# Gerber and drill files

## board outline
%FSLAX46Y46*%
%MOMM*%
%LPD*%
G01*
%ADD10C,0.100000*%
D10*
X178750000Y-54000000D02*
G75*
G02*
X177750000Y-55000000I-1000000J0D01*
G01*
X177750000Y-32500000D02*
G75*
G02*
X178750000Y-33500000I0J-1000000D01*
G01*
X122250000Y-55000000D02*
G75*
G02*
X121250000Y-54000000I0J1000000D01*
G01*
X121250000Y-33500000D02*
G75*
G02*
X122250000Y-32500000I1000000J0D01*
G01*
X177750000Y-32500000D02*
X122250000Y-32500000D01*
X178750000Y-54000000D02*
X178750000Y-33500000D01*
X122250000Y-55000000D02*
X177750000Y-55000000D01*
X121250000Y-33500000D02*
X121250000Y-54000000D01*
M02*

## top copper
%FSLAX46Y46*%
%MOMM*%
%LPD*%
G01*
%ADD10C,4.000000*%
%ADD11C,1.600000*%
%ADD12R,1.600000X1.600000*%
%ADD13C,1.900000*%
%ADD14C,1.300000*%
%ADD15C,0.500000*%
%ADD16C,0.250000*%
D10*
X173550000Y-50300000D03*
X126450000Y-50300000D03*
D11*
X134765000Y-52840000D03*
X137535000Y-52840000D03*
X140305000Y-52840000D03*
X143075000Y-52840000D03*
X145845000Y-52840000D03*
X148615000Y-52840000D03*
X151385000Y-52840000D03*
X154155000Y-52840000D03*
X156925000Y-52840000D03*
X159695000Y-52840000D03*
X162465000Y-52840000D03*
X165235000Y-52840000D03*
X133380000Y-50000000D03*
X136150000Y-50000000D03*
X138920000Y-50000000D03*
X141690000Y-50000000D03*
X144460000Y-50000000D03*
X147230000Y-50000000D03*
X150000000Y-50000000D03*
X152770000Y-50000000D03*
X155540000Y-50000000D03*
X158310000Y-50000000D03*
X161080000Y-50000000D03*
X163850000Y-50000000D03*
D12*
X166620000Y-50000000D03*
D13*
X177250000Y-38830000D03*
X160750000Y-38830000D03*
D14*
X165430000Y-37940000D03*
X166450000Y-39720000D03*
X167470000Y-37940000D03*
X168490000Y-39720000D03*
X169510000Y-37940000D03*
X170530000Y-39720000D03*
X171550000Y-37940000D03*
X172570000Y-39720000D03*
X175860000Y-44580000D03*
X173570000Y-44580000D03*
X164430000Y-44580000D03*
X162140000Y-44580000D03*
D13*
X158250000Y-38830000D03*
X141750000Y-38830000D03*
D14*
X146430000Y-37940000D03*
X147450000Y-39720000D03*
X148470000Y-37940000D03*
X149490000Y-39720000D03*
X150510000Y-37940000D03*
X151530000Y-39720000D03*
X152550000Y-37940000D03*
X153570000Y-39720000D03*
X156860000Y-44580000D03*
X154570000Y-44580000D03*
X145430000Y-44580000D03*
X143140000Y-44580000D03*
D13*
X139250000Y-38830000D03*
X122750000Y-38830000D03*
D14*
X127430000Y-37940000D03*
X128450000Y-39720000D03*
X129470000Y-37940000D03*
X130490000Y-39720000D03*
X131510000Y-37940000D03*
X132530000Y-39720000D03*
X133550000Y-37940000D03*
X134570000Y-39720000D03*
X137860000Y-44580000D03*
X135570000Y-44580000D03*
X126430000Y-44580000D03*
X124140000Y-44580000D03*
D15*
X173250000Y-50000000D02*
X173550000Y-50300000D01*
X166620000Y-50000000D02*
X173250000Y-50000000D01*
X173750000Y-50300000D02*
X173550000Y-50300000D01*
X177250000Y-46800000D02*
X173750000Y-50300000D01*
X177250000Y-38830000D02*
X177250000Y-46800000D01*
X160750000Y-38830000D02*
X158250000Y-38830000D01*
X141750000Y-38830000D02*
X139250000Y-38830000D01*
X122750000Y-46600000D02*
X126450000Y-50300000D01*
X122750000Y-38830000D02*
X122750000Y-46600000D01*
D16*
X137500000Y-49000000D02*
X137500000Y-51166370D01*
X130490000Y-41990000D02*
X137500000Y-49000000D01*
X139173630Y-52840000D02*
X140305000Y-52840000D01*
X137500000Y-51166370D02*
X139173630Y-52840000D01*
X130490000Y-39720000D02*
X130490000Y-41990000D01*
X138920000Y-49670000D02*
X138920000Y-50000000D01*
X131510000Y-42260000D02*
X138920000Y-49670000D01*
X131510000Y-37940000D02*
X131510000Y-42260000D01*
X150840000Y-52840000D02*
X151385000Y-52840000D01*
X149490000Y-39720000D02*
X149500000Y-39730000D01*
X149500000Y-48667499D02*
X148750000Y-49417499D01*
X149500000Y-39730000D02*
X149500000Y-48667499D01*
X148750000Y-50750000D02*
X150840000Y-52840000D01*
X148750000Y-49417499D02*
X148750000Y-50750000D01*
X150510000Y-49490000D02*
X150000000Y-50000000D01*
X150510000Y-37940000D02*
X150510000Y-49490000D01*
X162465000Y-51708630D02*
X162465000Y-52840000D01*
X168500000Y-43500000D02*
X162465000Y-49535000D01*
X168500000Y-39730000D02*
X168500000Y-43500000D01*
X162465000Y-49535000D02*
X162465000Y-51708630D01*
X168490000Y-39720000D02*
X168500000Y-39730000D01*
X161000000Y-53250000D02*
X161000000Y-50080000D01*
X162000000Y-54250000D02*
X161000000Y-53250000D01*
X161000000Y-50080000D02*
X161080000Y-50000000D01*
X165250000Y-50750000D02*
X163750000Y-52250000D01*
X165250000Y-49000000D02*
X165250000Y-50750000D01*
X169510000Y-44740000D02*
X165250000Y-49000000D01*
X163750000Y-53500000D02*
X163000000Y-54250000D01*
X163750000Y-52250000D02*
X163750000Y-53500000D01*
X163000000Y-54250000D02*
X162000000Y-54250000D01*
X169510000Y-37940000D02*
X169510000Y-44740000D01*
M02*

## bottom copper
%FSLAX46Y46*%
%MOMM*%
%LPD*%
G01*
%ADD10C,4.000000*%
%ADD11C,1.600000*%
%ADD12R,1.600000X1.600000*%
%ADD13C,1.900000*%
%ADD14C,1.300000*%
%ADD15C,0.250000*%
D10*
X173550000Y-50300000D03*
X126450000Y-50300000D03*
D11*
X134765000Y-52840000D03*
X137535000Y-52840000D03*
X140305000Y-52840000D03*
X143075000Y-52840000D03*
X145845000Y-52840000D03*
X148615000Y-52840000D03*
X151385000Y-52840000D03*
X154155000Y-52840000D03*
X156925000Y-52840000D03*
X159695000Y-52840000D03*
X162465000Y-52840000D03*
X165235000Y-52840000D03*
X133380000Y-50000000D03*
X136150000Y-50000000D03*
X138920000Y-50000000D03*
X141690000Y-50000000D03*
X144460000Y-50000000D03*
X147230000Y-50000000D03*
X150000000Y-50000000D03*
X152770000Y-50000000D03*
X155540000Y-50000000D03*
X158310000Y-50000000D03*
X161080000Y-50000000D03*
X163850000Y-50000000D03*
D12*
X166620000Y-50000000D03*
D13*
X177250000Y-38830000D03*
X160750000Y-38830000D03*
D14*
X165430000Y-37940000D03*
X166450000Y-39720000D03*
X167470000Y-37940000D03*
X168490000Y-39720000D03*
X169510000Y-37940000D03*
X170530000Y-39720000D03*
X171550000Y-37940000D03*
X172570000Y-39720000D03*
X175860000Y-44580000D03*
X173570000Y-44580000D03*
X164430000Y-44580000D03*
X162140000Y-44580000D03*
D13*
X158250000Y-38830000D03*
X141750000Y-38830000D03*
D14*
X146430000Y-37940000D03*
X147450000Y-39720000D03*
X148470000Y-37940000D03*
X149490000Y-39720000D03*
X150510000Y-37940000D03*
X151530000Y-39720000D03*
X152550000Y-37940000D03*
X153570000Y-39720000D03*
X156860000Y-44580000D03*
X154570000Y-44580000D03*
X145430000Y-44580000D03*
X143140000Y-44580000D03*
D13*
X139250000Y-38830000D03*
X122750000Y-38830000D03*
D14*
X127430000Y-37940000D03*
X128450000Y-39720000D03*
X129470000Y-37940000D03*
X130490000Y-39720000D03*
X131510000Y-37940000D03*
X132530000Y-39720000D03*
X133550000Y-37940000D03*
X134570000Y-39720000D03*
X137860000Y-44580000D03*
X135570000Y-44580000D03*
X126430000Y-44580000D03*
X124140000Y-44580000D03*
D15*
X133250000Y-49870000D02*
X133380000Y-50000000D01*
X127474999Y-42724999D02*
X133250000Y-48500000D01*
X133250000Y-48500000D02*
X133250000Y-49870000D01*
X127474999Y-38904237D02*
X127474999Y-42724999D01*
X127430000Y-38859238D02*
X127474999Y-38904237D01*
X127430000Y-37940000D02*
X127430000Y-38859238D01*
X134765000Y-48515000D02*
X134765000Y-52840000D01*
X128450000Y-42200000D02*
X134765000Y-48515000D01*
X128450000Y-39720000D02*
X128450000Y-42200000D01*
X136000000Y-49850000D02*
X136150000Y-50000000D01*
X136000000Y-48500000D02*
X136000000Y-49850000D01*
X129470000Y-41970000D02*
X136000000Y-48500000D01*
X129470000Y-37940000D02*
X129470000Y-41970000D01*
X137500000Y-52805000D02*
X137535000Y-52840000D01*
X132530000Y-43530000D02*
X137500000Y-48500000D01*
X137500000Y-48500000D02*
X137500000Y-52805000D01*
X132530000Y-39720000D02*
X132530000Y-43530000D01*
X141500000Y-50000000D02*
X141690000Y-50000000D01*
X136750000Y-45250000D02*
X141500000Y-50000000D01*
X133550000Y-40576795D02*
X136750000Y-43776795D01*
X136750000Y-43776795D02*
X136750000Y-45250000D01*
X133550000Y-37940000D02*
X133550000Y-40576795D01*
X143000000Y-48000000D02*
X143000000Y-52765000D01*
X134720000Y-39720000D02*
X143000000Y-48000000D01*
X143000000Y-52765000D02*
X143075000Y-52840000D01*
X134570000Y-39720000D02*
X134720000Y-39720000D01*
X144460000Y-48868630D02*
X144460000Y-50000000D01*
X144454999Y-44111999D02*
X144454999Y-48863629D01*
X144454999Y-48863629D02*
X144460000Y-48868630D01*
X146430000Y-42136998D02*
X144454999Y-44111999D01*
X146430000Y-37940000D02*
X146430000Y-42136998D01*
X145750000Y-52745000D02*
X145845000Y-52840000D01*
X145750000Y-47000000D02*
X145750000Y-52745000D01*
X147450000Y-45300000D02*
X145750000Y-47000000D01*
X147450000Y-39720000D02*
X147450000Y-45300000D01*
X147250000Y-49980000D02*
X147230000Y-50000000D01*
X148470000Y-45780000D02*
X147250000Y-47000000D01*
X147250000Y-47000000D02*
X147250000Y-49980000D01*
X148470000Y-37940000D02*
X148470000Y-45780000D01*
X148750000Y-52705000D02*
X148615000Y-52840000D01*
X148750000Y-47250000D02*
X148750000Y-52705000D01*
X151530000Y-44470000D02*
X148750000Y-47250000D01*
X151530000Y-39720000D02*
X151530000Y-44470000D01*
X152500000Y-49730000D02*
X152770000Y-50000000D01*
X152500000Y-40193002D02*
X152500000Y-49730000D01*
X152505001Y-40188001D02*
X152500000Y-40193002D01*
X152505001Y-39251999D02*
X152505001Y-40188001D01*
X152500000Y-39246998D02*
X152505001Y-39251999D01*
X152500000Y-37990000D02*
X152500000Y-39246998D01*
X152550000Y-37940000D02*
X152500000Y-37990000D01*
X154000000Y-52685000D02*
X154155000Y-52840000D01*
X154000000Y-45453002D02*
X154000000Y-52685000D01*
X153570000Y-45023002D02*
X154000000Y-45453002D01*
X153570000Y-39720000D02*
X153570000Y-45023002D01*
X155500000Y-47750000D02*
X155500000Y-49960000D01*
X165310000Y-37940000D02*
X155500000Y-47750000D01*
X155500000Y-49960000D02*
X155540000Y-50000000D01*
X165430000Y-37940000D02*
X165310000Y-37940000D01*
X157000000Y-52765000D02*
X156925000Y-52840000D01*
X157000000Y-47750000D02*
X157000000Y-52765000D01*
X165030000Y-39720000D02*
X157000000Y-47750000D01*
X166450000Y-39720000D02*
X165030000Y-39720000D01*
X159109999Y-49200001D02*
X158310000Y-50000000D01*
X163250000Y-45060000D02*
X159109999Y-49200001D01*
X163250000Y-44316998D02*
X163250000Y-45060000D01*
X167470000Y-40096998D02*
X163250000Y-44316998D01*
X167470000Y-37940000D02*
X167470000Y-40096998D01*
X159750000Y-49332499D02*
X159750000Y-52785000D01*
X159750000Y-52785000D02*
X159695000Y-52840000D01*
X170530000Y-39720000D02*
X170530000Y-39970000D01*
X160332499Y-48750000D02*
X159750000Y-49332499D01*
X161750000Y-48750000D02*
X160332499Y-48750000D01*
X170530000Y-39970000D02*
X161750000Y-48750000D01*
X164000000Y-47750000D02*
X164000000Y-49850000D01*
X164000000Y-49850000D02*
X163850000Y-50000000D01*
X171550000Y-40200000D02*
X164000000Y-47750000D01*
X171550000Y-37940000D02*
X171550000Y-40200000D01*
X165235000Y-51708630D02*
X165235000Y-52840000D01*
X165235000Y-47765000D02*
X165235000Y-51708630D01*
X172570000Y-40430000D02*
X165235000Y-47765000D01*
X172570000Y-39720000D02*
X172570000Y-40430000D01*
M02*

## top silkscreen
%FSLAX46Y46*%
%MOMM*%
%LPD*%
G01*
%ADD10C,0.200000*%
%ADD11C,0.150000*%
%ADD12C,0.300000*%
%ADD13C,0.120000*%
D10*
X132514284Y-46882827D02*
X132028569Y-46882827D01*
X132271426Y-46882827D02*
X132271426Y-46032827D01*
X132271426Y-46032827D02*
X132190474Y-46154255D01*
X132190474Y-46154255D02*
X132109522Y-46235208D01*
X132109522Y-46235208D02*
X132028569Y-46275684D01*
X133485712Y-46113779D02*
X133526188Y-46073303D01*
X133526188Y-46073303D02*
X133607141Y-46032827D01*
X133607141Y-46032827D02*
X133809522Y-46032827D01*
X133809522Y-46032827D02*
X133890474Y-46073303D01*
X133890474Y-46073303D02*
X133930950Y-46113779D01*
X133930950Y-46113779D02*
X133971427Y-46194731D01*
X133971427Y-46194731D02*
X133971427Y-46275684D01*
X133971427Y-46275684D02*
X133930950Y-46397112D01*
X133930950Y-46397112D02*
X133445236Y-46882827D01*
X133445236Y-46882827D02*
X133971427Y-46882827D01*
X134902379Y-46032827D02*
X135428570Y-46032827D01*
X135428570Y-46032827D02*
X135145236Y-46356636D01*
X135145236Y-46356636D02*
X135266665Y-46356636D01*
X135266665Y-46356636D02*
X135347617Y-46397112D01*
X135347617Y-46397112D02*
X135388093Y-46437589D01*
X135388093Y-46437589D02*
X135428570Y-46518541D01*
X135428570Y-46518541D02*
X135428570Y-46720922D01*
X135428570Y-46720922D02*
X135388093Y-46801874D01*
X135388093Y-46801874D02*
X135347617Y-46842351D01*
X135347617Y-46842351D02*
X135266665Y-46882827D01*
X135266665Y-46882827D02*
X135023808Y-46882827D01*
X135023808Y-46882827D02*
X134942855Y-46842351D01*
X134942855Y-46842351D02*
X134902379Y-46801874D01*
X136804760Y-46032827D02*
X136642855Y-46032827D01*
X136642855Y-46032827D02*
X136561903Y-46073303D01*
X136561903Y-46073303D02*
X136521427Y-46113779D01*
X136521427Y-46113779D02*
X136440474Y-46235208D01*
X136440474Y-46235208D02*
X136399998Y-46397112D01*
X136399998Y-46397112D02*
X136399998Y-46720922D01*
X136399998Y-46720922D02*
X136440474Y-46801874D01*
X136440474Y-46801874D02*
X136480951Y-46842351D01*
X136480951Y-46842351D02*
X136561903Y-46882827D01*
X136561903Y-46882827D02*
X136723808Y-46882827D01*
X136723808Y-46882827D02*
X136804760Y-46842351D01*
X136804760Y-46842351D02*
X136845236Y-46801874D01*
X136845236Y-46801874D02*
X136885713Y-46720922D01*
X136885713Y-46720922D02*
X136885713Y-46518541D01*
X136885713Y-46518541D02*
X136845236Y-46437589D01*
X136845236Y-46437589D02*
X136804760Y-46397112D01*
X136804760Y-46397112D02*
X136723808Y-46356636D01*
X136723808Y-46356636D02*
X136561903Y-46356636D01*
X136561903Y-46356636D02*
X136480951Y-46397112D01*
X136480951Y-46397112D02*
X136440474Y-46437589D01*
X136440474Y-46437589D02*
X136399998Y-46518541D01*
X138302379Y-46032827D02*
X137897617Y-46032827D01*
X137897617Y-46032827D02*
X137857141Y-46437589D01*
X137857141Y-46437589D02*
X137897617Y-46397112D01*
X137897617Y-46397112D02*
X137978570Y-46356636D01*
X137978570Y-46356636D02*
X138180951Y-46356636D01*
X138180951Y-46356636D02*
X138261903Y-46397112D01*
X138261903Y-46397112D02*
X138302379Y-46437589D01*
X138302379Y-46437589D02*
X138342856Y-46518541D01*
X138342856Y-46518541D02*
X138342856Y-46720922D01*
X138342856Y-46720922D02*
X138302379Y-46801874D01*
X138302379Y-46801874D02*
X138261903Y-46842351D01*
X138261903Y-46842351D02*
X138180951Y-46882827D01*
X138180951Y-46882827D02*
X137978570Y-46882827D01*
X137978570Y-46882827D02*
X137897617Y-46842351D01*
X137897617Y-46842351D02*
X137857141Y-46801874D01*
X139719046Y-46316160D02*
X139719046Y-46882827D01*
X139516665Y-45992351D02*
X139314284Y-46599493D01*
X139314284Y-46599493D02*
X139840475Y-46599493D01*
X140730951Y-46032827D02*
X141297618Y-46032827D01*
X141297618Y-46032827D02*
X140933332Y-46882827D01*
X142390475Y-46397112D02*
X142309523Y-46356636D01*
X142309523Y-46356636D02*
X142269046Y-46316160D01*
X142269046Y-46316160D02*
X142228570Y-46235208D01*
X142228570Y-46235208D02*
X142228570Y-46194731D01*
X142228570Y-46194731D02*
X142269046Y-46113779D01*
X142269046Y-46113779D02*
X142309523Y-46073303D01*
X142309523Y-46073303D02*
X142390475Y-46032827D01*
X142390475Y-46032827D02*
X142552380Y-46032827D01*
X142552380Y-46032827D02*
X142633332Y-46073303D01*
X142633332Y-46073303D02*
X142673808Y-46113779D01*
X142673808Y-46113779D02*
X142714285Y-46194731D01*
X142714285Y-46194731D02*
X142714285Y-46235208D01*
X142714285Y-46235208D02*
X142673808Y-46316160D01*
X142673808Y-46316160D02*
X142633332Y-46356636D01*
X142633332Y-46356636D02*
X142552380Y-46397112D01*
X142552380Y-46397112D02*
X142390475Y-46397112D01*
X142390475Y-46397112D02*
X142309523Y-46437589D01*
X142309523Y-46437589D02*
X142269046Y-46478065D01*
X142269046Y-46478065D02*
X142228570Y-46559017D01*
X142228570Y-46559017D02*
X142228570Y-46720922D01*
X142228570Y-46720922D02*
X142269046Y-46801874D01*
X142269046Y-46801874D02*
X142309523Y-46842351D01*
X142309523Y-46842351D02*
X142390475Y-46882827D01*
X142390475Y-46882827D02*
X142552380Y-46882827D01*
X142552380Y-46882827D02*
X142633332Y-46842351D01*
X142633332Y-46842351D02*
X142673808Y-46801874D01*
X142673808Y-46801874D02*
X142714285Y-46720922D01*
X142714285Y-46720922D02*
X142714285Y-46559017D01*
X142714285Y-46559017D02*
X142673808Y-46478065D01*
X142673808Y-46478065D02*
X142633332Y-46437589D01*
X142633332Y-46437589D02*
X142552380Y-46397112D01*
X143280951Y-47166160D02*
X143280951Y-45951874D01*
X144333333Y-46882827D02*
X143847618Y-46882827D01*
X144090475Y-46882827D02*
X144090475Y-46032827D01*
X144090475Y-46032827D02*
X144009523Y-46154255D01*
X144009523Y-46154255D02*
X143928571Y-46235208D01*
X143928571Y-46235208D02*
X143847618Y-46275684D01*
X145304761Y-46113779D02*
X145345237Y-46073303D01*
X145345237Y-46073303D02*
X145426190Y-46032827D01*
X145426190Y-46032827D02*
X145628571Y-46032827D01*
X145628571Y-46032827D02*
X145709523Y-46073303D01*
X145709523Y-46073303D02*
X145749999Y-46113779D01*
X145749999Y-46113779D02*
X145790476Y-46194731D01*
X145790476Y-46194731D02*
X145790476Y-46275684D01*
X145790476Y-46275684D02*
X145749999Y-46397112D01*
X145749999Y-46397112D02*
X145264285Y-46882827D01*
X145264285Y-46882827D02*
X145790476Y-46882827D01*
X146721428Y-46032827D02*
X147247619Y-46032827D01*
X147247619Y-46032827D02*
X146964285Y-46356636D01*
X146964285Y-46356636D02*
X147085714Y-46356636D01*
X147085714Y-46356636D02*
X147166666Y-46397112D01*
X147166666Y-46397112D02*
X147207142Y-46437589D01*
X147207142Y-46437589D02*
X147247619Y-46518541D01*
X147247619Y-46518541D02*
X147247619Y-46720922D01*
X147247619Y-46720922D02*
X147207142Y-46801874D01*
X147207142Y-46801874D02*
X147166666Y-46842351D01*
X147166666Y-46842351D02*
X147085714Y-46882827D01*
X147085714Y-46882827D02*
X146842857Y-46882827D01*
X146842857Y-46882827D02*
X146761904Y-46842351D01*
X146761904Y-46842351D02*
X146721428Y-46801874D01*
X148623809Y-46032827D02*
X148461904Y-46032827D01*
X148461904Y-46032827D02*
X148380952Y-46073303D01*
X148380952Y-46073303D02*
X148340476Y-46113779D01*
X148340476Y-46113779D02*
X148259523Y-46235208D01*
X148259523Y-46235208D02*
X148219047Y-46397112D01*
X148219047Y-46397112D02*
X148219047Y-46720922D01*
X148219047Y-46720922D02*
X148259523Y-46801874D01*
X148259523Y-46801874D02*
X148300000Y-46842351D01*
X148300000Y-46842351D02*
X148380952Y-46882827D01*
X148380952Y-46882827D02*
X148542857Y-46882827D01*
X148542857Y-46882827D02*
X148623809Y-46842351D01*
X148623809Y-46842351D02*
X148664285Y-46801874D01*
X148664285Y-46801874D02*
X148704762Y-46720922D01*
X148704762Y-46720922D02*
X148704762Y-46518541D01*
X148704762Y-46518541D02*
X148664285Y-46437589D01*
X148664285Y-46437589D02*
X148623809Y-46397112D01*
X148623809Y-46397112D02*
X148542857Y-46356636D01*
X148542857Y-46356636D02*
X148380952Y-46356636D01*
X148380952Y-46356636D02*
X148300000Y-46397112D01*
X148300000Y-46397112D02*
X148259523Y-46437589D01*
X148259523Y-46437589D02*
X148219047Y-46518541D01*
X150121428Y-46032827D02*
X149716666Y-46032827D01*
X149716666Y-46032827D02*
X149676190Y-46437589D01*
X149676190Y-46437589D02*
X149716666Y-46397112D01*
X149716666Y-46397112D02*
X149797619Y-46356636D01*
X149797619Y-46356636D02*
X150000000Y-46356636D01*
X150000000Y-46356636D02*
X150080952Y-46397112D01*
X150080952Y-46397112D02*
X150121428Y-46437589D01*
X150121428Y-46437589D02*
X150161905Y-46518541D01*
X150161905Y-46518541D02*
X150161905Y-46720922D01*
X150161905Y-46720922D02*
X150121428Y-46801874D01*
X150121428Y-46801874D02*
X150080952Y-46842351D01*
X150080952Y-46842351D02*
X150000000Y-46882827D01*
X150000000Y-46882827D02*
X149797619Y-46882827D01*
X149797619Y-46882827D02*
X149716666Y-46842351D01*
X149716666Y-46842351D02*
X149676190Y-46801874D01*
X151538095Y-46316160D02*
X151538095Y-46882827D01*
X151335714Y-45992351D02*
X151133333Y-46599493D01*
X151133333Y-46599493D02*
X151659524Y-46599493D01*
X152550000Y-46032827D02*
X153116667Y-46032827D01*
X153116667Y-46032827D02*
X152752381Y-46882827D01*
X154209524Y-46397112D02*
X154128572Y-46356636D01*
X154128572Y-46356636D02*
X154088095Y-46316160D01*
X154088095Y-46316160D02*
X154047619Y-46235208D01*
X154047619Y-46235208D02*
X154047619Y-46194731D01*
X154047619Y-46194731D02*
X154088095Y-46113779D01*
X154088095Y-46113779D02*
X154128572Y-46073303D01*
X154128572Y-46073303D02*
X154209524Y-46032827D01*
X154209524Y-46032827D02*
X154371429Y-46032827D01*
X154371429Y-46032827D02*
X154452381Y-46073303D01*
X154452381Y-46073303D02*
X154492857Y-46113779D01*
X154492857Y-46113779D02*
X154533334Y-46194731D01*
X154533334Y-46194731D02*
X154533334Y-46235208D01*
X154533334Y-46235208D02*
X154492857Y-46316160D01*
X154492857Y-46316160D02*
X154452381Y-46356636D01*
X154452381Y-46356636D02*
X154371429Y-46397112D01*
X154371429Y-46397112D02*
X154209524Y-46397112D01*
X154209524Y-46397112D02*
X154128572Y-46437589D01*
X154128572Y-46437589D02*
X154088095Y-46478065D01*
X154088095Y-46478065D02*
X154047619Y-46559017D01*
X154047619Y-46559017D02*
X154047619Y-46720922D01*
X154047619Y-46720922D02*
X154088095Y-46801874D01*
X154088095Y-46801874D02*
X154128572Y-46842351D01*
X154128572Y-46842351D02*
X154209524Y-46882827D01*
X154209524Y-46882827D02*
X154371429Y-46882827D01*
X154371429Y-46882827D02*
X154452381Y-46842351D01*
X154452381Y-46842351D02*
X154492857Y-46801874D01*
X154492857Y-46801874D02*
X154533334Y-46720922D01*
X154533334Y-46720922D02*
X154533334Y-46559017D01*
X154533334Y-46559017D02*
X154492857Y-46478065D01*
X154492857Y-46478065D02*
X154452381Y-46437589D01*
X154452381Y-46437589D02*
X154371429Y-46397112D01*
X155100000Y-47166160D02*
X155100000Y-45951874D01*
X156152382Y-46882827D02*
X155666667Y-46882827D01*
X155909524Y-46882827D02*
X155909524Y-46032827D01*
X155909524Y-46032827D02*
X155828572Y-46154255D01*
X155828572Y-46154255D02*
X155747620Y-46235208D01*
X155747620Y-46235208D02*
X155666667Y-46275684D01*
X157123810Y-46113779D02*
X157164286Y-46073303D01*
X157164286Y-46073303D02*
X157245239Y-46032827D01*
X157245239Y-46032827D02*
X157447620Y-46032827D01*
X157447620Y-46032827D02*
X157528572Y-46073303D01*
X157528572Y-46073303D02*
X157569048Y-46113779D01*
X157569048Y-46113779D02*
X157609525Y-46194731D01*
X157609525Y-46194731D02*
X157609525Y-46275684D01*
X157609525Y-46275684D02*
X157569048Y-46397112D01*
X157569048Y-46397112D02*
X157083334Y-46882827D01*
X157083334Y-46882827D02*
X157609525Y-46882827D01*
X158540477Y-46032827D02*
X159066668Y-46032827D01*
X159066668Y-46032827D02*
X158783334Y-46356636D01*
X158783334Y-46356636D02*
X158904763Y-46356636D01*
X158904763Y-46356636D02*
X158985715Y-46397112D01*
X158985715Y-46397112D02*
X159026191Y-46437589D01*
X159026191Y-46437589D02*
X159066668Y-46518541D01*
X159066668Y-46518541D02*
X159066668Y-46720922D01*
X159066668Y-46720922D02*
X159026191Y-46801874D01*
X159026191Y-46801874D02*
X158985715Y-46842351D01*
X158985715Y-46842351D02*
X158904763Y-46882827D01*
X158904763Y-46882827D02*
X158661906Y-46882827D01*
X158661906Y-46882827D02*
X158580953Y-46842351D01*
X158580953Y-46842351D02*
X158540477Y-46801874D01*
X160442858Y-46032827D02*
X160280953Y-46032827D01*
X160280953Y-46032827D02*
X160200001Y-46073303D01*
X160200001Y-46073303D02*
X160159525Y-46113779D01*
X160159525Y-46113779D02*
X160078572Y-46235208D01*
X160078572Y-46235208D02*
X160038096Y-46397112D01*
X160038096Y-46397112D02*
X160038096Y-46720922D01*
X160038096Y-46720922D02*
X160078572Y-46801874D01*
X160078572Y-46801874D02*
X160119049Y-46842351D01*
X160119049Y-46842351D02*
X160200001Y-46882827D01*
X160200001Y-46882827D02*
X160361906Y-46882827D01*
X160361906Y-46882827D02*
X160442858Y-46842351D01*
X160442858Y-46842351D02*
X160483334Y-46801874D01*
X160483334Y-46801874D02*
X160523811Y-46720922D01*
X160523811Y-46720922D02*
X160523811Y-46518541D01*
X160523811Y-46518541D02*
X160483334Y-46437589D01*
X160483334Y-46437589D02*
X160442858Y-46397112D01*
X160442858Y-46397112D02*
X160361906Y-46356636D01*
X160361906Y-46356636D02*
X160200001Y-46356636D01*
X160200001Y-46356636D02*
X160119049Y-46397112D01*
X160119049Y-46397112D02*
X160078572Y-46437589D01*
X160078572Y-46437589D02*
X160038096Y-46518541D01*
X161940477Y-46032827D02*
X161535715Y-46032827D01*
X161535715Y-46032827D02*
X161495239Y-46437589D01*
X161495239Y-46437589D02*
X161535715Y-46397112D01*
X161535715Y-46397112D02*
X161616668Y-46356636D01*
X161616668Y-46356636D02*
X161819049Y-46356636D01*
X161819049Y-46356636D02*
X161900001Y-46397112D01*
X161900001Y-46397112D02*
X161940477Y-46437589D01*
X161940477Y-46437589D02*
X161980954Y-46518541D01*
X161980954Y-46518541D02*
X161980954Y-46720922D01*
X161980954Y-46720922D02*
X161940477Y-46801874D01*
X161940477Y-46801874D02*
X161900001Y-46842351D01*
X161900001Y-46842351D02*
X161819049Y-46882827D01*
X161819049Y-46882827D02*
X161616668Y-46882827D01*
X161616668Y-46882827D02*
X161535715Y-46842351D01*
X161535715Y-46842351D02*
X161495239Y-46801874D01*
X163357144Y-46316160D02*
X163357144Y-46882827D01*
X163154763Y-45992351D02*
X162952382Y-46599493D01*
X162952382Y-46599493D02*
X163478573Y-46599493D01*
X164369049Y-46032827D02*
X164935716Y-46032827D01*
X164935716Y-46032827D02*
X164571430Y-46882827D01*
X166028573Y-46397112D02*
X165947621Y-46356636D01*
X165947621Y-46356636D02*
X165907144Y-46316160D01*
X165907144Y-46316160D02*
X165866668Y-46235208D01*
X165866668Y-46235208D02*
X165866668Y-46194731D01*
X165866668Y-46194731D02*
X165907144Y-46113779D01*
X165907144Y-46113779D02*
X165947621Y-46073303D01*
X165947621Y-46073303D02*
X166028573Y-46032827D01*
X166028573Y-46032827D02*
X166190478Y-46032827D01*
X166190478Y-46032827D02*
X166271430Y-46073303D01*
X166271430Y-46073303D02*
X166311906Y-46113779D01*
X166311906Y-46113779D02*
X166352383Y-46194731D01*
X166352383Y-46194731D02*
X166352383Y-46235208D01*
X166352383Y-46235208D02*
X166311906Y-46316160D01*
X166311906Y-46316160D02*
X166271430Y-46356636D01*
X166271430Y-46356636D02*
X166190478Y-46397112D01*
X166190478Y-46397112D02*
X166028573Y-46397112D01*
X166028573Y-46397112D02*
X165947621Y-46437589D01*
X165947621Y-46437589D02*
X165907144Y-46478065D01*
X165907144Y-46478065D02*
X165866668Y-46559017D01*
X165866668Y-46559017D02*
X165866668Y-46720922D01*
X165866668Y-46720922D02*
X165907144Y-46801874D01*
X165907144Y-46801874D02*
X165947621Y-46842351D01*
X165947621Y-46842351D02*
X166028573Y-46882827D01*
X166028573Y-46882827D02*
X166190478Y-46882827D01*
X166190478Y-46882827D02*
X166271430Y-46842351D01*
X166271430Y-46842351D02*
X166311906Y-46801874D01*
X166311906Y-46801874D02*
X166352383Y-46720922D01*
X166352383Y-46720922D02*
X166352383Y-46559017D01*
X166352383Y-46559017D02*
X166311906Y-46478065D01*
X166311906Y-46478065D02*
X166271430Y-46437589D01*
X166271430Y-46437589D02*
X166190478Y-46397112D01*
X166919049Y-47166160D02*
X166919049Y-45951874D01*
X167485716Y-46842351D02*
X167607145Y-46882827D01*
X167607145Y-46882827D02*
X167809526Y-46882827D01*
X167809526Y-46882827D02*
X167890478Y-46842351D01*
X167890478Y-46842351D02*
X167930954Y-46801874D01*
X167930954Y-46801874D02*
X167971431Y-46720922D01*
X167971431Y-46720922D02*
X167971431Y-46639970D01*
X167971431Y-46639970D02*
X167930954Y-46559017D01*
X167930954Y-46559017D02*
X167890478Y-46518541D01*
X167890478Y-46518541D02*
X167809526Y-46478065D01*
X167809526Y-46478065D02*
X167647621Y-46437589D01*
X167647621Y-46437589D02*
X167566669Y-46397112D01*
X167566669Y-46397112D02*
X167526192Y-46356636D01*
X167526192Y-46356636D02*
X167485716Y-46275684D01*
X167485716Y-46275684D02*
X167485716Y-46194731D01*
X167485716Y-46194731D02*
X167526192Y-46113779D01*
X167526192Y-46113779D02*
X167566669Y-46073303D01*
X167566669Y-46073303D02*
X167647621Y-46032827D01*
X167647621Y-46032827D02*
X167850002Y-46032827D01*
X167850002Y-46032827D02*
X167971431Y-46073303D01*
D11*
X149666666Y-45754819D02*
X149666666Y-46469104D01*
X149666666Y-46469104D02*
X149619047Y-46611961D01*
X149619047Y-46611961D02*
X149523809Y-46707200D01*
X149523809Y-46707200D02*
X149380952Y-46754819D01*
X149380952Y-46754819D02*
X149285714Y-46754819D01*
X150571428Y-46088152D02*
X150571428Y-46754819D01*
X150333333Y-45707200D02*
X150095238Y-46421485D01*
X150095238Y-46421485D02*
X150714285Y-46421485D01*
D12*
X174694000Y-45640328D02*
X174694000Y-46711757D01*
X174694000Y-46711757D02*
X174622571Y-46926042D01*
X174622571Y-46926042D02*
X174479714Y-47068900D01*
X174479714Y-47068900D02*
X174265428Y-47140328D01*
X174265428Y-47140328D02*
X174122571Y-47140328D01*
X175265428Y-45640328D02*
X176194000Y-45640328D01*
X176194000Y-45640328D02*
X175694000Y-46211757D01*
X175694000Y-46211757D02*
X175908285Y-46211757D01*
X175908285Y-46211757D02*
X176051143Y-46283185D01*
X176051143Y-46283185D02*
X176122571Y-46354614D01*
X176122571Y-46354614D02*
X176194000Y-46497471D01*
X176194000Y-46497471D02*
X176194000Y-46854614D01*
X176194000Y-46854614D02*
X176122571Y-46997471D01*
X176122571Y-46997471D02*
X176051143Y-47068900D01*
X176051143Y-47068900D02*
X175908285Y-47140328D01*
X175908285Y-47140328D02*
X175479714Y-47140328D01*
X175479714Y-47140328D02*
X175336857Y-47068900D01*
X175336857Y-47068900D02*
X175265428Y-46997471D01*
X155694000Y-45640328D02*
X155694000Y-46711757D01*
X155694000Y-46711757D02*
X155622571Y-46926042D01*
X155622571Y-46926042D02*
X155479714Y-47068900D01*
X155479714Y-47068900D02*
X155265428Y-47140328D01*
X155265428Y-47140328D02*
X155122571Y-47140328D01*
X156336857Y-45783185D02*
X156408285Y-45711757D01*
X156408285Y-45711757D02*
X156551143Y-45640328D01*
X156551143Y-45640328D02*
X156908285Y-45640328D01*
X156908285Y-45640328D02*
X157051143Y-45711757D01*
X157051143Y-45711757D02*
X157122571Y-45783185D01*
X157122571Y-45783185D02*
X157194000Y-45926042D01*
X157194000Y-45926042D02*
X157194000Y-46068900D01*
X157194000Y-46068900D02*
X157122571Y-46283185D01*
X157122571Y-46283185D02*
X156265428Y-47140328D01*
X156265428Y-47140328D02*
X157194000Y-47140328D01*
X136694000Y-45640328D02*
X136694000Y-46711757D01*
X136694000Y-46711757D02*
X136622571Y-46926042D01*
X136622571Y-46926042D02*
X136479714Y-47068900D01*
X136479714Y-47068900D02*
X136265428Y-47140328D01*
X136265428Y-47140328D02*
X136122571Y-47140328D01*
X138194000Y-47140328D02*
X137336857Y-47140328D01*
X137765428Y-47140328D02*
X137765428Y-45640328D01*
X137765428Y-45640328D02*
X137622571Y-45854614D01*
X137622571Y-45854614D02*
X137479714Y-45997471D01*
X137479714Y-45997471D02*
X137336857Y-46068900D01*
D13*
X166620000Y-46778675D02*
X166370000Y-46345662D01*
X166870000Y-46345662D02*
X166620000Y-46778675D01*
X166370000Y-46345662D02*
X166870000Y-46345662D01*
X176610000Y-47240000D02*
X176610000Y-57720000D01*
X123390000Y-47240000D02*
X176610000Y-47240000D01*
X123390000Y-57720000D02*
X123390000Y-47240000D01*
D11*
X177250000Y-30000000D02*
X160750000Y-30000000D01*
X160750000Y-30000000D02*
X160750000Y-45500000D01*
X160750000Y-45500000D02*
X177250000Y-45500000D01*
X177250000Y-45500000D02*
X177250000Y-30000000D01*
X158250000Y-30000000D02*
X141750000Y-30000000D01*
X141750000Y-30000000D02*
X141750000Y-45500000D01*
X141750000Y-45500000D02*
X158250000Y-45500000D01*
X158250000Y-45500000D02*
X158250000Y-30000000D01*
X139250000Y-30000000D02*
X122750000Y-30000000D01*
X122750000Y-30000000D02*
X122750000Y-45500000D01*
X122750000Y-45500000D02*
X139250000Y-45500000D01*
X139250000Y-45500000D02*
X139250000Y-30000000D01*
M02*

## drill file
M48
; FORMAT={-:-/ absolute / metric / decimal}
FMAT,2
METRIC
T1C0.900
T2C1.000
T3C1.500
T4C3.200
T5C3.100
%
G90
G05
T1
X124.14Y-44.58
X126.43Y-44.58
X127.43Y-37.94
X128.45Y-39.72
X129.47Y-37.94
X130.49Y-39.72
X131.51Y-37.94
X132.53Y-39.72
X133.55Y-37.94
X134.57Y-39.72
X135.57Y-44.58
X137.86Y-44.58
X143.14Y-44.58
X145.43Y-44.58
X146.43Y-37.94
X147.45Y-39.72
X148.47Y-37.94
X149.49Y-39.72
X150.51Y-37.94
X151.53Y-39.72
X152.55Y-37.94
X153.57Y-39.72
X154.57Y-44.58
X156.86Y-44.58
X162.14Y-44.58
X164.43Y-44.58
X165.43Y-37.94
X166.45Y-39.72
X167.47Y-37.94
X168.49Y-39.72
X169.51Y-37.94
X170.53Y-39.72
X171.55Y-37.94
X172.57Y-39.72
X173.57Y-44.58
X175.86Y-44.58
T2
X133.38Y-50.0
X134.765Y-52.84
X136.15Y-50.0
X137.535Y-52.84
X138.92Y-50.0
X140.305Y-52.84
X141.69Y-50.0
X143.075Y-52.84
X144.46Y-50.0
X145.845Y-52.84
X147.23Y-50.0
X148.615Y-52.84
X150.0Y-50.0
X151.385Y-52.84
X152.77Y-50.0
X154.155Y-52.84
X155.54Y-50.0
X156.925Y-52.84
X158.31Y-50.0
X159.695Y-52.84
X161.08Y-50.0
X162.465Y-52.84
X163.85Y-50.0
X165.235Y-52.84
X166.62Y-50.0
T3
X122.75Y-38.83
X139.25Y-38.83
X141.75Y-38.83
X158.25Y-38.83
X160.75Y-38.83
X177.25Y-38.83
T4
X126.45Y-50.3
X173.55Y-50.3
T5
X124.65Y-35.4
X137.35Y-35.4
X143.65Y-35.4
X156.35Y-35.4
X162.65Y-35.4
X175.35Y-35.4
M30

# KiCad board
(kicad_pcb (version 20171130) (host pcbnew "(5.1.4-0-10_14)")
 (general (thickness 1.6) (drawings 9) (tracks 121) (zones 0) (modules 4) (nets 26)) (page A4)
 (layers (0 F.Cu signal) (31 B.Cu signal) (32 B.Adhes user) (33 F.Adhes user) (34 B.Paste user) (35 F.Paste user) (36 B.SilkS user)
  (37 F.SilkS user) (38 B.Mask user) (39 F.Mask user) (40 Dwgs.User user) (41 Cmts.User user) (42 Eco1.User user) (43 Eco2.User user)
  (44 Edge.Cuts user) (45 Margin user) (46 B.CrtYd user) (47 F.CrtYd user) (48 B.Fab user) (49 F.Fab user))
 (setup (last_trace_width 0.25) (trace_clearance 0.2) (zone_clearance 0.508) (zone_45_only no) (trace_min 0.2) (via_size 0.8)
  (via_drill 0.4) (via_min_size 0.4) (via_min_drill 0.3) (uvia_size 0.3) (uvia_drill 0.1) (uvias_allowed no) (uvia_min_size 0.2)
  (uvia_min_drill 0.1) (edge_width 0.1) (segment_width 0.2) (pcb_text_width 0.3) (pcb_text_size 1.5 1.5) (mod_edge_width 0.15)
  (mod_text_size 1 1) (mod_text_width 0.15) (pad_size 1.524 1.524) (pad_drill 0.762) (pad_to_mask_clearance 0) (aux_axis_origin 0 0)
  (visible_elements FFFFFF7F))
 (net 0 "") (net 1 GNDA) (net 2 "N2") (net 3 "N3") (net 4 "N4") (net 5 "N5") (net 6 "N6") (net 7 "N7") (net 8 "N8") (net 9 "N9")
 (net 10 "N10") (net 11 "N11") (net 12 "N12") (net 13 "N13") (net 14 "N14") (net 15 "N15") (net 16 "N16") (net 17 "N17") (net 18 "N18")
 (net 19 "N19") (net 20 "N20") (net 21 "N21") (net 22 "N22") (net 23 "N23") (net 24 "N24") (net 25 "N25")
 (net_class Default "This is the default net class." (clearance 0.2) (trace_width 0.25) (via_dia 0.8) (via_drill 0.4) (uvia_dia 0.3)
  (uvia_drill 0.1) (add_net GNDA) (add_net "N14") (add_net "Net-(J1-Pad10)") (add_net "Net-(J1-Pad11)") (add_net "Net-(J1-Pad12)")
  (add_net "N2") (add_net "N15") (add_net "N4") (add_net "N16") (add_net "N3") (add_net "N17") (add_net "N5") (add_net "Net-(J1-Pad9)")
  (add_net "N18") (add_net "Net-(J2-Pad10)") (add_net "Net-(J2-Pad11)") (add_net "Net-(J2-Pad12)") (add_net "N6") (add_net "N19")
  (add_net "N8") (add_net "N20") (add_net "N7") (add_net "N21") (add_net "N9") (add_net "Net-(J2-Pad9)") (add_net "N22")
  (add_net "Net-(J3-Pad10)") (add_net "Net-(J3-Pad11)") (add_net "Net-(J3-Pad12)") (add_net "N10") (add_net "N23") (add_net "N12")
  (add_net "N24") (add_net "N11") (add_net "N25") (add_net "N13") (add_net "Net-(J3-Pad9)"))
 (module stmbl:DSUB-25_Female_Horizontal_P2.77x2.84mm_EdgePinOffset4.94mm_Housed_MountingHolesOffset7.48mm (layer F.Cu) (at 166.62 50)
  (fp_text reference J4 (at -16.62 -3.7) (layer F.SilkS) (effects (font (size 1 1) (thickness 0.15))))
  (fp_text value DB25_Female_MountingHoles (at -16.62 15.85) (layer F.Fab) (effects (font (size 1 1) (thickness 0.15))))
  (fp_line (start 0 -3.221325) (end -0.25 -3.654338) (layer F.SilkS) (width 0.12))
  (fp_line (start 0.25 -3.654338) (end 0 -3.221325) (layer F.SilkS) (width 0.12))
  (fp_line (start -0.25 -3.654338) (end 0.25 -3.654338) (layer F.SilkS) (width 0.12))
  (fp_line (start 9.99 -2.76) (end 9.99 7.72) (layer F.SilkS) (width 0.12))
  (fp_line (start -43.23 -2.76) (end 9.99 -2.76) (layer F.SilkS) (width 0.12))
  (fp_line (start -43.23 7.72) (end -43.23 -2.76) (layer F.SilkS) (width 0.12))
  (pad 0 thru_hole circle (at 6.93 0.3) (size 4 4) (drill 3.2) (layers *.Cu *.Mask) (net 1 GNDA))
  (pad 0 thru_hole circle (at -40.17 0.3) (size 4 4) (drill 3.2) (layers *.Cu *.Mask) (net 1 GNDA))
  (pad 25 thru_hole circle (at -31.855 2.84) (size 1.6 1.6) (drill 1) (layers *.Cu *.Mask) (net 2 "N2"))
  (pad 24 thru_hole circle (at -29.085 2.84) (size 1.6 1.6) (drill 1) (layers *.Cu *.Mask) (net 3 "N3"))
  (pad 23 thru_hole circle (at -26.315 2.84) (size 1.6 1.6) (drill 1) (layers *.Cu *.Mask) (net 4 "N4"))
  (pad 22 thru_hole circle (at -23.545 2.84) (size 1.6 1.6) (drill 1) (layers *.Cu *.Mask) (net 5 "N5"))
  (pad 21 thru_hole circle (at -20.775 2.84) (size 1.6 1.6) (drill 1) (layers *.Cu *.Mask) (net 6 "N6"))
  (pad 20 thru_hole circle (at -18.005 2.84) (size 1.6 1.6) (drill 1) (layers *.Cu *.Mask) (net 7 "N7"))
  (pad 19 thru_hole circle (at -15.235 2.84) (size 1.6 1.6) (drill 1) (layers *.Cu *.Mask) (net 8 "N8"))
  (pad 18 thru_hole circle (at -12.465 2.84) (size 1.6 1.6) (drill 1) (layers *.Cu *.Mask) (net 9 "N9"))
  (pad 17 thru_hole circle (at -9.695 2.84) (size 1.6 1.6) (drill 1) (layers *.Cu *.Mask) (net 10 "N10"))
  (pad 16 thru_hole circle (at -6.925 2.84) (size 1.6 1.6) (drill 1) (layers *.Cu *.Mask) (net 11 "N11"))
  (pad 15 thru_hole circle (at -4.155 2.84) (size 1.6 1.6) (drill 1) (layers *.Cu *.Mask) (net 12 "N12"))
  (pad 14 thru_hole circle (at -1.385 2.84) (size 1.6 1.6) (drill 1) (layers *.Cu *.Mask) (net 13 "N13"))
  (pad 13 thru_hole circle (at -33.24 0) (size 1.6 1.6) (drill 1) (layers *.Cu *.Mask) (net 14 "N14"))
  (pad 12 thru_hole circle (at -30.47 0) (size 1.6 1.6) (drill 1) (layers *.Cu *.Mask) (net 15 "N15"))
  (pad 11 thru_hole circle (at -27.7 0) (size 1.6 1.6) (drill 1) (layers *.Cu *.Mask) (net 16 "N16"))
  (pad 10 thru_hole circle (at -24.93 0) (size 1.6 1.6) (drill 1) (layers *.Cu *.Mask) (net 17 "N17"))
  (pad 9 thru_hole circle (at -22.16 0) (size 1.6 1.6) (drill 1) (layers *.Cu *.Mask) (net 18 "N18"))
  (pad 8 thru_hole circle (at -19.39 0) (size 1.6 1.6) (drill 1) (layers *.Cu *.Mask) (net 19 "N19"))
  (pad 7 thru_hole circle (at -16.62 0) (size 1.6 1.6) (drill 1) (layers *.Cu *.Mask) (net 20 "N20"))
  (pad 6 thru_hole circle (at -13.85 0) (size 1.6 1.6) (drill 1) (layers *.Cu *.Mask) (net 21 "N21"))
  (pad 5 thru_hole circle (at -11.08 0) (size 1.6 1.6) (drill 1) (layers *.Cu *.Mask) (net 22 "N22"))
  (pad 4 thru_hole circle (at -8.31 0) (size 1.6 1.6) (drill 1) (layers *.Cu *.Mask) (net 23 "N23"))
  (pad 3 thru_hole circle (at -5.54 0) (size 1.6 1.6) (drill 1) (layers *.Cu *.Mask) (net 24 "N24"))
  (pad 2 thru_hole circle (at -2.77 0) (size 1.6 1.6) (drill 1) (layers *.Cu *.Mask) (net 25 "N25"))
  (pad 1 thru_hole rect (at 0 0) (size 1.6 1.6) (drill 1) (layers *.Cu *.Mask) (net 1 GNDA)))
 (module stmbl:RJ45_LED (layer F.Cu) (at 169 30)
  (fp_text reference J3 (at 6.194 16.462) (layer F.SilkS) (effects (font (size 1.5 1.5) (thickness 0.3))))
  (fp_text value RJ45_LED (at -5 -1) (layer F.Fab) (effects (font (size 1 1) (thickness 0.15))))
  (fp_line (start 8.25 0) (end -8.25 0) (layer F.SilkS) (width 0.15))
  (fp_line (start -8.25 0) (end -8.25 15.5) (layer F.SilkS) (width 0.15))
  (fp_line (start -8.25 15.5) (end 8.25 15.5) (layer F.SilkS) (width 0.15))
  (fp_line (start 8.25 15.5) (end 8.25 0) (layer F.SilkS) (width 0.15))
  (pad "" np_thru_hole circle (at 6.35 5.4) (size 3.1 3.1) (drill 3.1) (layers *.Cu *.Mask) (clearance 0.5))
  (pad "" np_thru_hole circle (at -6.35 5.4) (size 3.1 3.1) (drill 3.1) (layers *.Cu *.Mask) (clearance 0.5))
  (pad 13 thru_hole circle (at 8.25 8.83) (size 1.9 1.9) (drill 1.5) (layers *.Cu *.Mask) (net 1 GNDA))
  (pad 13 thru_hole circle (at -8.25 8.83) (size 1.9 1.9) (drill 1.5) (layers *.Cu *.Mask) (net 1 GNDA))
  (pad 1 thru_hole circle (at -3.57 7.94) (size 1.3 1.3) (drill 0.9) (layers *.Cu *.Mask) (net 22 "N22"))
  (pad 2 thru_hole circle (at -2.55 9.72) (size 1.3 1.3) (drill 0.9) (layers *.Cu *.Mask) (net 10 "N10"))
  (pad 3 thru_hole circle (at -1.53 7.94) (size 1.3 1.3) (drill 0.9) (layers *.Cu *.Mask) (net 23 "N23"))
  (pad 4 thru_hole circle (at -0.51 9.72) (size 1.3 1.3) (drill 0.9) (layers *.Cu *.Mask) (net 12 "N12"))
  (pad 5 thru_hole circle (at 0.51 7.94) (size 1.3 1.3) (drill 0.9) (layers *.Cu *.Mask) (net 24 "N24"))
  (pad 6 thru_hole circle (at 1.53 9.72) (size 1.3 1.3) (drill 0.9) (layers *.Cu *.Mask) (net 11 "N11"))
  (pad 7 thru_hole circle (at 2.55 7.94) (size 1.3 1.3) (drill 0.9) (layers *.Cu *.Mask) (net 25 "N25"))
  (pad 8 thru_hole circle (at 3.57 9.72) (size 1.3 1.3) (drill 0.9) (layers *.Cu *.Mask) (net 13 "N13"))
  (pad 10 thru_hole circle (at 6.86 14.58) (size 1.3 1.3) (drill 0.9) (layers *.Cu *.Mask))
  (pad 9 thru_hole circle (at 4.57 14.58) (size 1.3 1.3) (drill 0.9) (layers *.Cu *.Mask))
  (pad 12 thru_hole circle (at -4.57 14.58) (size 1.3 1.3) (drill 0.9) (layers *.Cu *.Mask))
  (pad 11 thru_hole circle (at -6.86 14.58) (size 1.3 1.3) (drill 0.9) (layers *.Cu *.Mask)))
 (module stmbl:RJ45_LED (layer F.Cu) (at 150 30)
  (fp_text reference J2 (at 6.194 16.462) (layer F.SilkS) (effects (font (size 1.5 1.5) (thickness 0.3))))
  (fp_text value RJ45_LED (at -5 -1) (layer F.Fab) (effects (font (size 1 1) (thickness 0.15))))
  (fp_line (start 8.25 0) (end -8.25 0) (layer F.SilkS) (width 0.15))
  (fp_line (start -8.25 0) (end -8.25 15.5) (layer F.SilkS) (width 0.15))
  (fp_line (start -8.25 15.5) (end 8.25 15.5) (layer F.SilkS) (width 0.15))
  (fp_line (start 8.25 15.5) (end 8.25 0) (layer F.SilkS) (width 0.15))
  (pad "" np_thru_hole circle (at 6.35 5.4) (size 3.1 3.1) (drill 3.1) (layers *.Cu *.Mask) (clearance 0.5))
  (pad "" np_thru_hole circle (at -6.35 5.4) (size 3.1 3.1) (drill 3.1) (layers *.Cu *.Mask) (clearance 0.5))
  (pad 13 thru_hole circle (at 8.25 8.83) (size 1.9 1.9) (drill 1.5) (layers *.Cu *.Mask) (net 1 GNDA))
  (pad 13 thru_hole circle (at -8.25 8.83) (size 1.9 1.9) (drill 1.5) (layers *.Cu *.Mask) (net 1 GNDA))
  (pad 1 thru_hole circle (at -3.57 7.94) (size 1.3 1.3) (drill 0.9) (layers *.Cu *.Mask) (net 18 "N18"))
  (pad 2 thru_hole circle (at -2.55 9.72) (size 1.3 1.3) (drill 0.9) (layers *.Cu *.Mask) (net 6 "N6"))
  (pad 3 thru_hole circle (at -1.53 7.94) (size 1.3 1.3) (drill 0.9) (layers *.Cu *.Mask) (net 19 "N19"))
  (pad 4 thru_hole circle (at -0.51 9.72) (size 1.3 1.3) (drill 0.9) (layers *.Cu *.Mask) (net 8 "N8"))
  (pad 5 thru_hole circle (at 0.51 7.94) (size 1.3 1.3) (drill 0.9) (layers *.Cu *.Mask) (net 20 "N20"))
  (pad 6 thru_hole circle (at 1.53 9.72) (size 1.3 1.3) (drill 0.9) (layers *.Cu *.Mask) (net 7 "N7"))
  (pad 7 thru_hole circle (at 2.55 7.94) (size 1.3 1.3) (drill 0.9) (layers *.Cu *.Mask) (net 21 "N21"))
  (pad 8 thru_hole circle (at 3.57 9.72) (size 1.3 1.3) (drill 0.9) (layers *.Cu *.Mask) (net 9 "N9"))
  (pad 10 thru_hole circle (at 6.86 14.58) (size 1.3 1.3) (drill 0.9) (layers *.Cu *.Mask))
  (pad 9 thru_hole circle (at 4.57 14.58) (size 1.3 1.3) (drill 0.9) (layers *.Cu *.Mask))
  (pad 12 thru_hole circle (at -4.57 14.58) (size 1.3 1.3) (drill 0.9) (layers *.Cu *.Mask))
  (pad 11 thru_hole circle (at -6.86 14.58) (size 1.3 1.3) (drill 0.9) (layers *.Cu *.Mask)))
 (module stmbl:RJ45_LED (layer F.Cu) (at 131 30)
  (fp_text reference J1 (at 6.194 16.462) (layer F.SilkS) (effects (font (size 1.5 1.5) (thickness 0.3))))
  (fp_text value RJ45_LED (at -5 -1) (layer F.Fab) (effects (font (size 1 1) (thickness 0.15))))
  (fp_line (start 8.25 0) (end -8.25 0) (layer F.SilkS) (width 0.15))
  (fp_line (start -8.25 0) (end -8.25 15.5) (layer F.SilkS) (width 0.15))
  (fp_line (start -8.25 15.5) (end 8.25 15.5) (layer F.SilkS) (width 0.15))
  (fp_line (start 8.25 15.5) (end 8.25 0) (layer F.SilkS) (width 0.15))
  (pad "" np_thru_hole circle (at 6.35 5.4) (size 3.1 3.1) (drill 3.1) (layers *.Cu *.Mask) (clearance 0.5))
  (pad "" np_thru_hole circle (at -6.35 5.4) (size 3.1 3.1) (drill 3.1) (layers *.Cu *.Mask) (clearance 0.5))
  (pad 13 thru_hole circle (at 8.25 8.83) (size 1.9 1.9) (drill 1.5) (layers *.Cu *.Mask) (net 1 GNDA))
  (pad 13 thru_hole circle (at -8.25 8.83) (size 1.9 1.9) (drill 1.5) (layers *.Cu *.Mask) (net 1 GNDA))
  (pad 1 thru_hole circle (at -3.57 7.94) (size 1.3 1.3) (drill 0.9) (layers *.Cu *.Mask) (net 14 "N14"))
  (pad 2 thru_hole circle (at -2.55 9.72) (size 1.3 1.3) (drill 0.9) (layers *.Cu *.Mask) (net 2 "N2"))
  (pad 3 thru_hole circle (at -1.53 7.94) (size 1.3 1.3) (drill 0.9) (layers *.Cu *.Mask) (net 15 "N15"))
  (pad 4 thru_hole circle (at -0.51 9.72) (size 1.3 1.3) (drill 0.9) (layers *.Cu *.Mask) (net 4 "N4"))
  (pad 5 thru_hole circle (at 0.51 7.94) (size 1.3 1.3) (drill 0.9) (layers *.Cu *.Mask) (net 16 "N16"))
  (pad 6 thru_hole circle (at 1.53 9.72) (size 1.3 1.3) (drill 0.9) (layers *.Cu *.Mask) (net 3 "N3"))
  (pad 7 thru_hole circle (at 2.55 7.94) (size 1.3 1.3) (drill 0.9) (layers *.Cu *.Mask) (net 17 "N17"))
  (pad 8 thru_hole circle (at 3.57 9.72) (size 1.3 1.3) (drill 0.9) (layers *.Cu *.Mask) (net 5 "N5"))
  (pad 10 thru_hole circle (at 6.86 14.58) (size 1.3 1.3) (drill 0.9) (layers *.Cu *.Mask))
  (pad 9 thru_hole circle (at 4.57 14.58) (size 1.3 1.3) (drill 0.9) (layers *.Cu *.Mask))
  (pad 12 thru_hole circle (at -4.57 14.58) (size 1.3 1.3) (drill 0.9) (layers *.Cu *.Mask))
  (pad 11 thru_hole circle (at -6.86 14.58) (size 1.3 1.3) (drill 0.9) (layers *.Cu *.Mask)))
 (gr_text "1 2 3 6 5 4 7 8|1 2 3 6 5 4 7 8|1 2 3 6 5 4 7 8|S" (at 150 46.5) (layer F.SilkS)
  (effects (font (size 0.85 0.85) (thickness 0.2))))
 (gr_arc (start 177.75 54) (end 177.75 55) (angle -90) (layer Edge.Cuts) (width 0.1))
 (gr_arc (start 177.75 33.5) (end 178.75 33.5) (angle -90) (layer Edge.Cuts) (width 0.1))
 (gr_arc (start 122.25 54) (end 121.25 54) (angle -90) (layer Edge.Cuts) (width 0.1))
 (gr_arc (start 122.25 33.5) (end 122.25 32.5) (angle -90) (layer Edge.Cuts) (width 0.1))
 (gr_line (start 177.75 32.5) (end 122.25 32.5) (layer Edge.Cuts) (width 0.1))
 (gr_line (start 178.75 54) (end 178.75 33.5) (layer Edge.Cuts) (width 0.1))
 (gr_line (start 122.25 55) (end 177.75 55) (layer Edge.Cuts) (width 0.1))
 (gr_line (start 121.25 33.5) (end 121.25 54) (layer Edge.Cuts) (width 0.1))
 (segment (start 173.25 50) (end 173.55 50.3) (width 0.5) (layer F.Cu) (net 1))
 (segment (start 166.62 50) (end 173.25 50) (width 0.5) (layer F.Cu) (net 1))
 (segment (start 173.75 50.3) (end 173.55 50.3) (width 0.5) (layer F.Cu) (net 1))
 (segment (start 177.25 46.8) (end 173.75 50.3) (width 0.5) (layer F.Cu) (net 1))
 (segment (start 177.25 38.83) (end 177.25 46.8) (width 0.5) (layer F.Cu) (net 1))
 (segment (start 160.75 38.83) (end 158.25 38.83) (width 0.5) (layer F.Cu) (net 1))
 (segment (start 141.75 38.83) (end 139.25 38.83) (width 0.5) (layer F.Cu) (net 1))
 (segment (start 122.75 46.6) (end 126.45 50.3) (width 0.5) (layer F.Cu) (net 1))
 (segment (start 122.75 38.83) (end 122.75 46.6) (width 0.5) (layer F.Cu) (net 1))
 (segment (start 133.25 49.87) (end 133.38 50) (width 0.25) (layer B.Cu) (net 14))
 (segment (start 127.474999 42.724999) (end 133.25 48.5) (width 0.25) (layer B.Cu) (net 14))
 (segment (start 133.25 48.5) (end 133.25 49.87) (width 0.25) (layer B.Cu) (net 14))
 (segment (start 127.474999 38.904237) (end 127.474999 42.724999) (width 0.25) (layer B.Cu) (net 14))
 (segment (start 127.43 38.859238) (end 127.474999 38.904237) (width 0.25) (layer B.Cu) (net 14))
 (segment (start 127.43 37.94) (end 127.43 38.859238) (width 0.25) (layer B.Cu) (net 14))
 (segment (start 134.765 48.515) (end 134.765 52.84) (width 0.25) (layer B.Cu) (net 2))
 (segment (start 128.45 42.2) (end 134.765 48.515) (width 0.25) (layer B.Cu) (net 2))
 (segment (start 128.45 39.72) (end 128.45 42.2) (width 0.25) (layer B.Cu) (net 2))
 (segment (start 136 49.85) (end 136.15 50) (width 0.25) (layer B.Cu) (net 15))
 (segment (start 136 48.5) (end 136 49.85) (width 0.25) (layer B.Cu) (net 15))
 (segment (start 129.47 41.97) (end 136 48.5) (width 0.25) (layer B.Cu) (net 15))
 (segment (start 129.47 37.94) (end 129.47 41.97) (width 0.25) (layer B.Cu) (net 15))
 (segment (start 137.5 49) (end 137.5 51.16637) (width 0.25) (layer F.Cu) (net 4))
 (segment (start 130.49 41.99) (end 137.5 49) (width 0.25) (layer F.Cu) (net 4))
 (segment (start 139.17363 52.84) (end 140.305 52.84) (width 0.25) (layer F.Cu) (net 4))
 (segment (start 137.5 51.16637) (end 139.17363 52.84) (width 0.25) (layer F.Cu) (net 4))
 (segment (start 130.49 39.72) (end 130.49 41.99) (width 0.25) (layer F.Cu) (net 4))
 (segment (start 138.92 49.67) (end 138.92 50) (width 0.25) (layer F.Cu) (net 16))
 (segment (start 131.51 42.26) (end 138.92 49.67) (width 0.25) (layer F.Cu) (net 16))
 (segment (start 131.51 37.94) (end 131.51 42.26) (width 0.25) (layer F.Cu) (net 16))
 (segment (start 137.5 52.805) (end 137.535 52.84) (width 0.25) (layer B.Cu) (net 3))
 (segment (start 132.53 43.53) (end 137.5 48.5) (width 0.25) (layer B.Cu) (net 3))
 (segment (start 137.5 48.5) (end 137.5 52.805) (width 0.25) (layer B.Cu) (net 3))
 (segment (start 132.53 39.72) (end 132.53 43.53) (width 0.25) (layer B.Cu) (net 3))
 (segment (start 141.5 50) (end 141.69 50) (width 0.25) (layer B.Cu) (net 17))
 (segment (start 136.75 45.25) (end 141.5 50) (width 0.25) (layer B.Cu) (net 17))
 (segment (start 133.55 40.576795) (end 136.75 43.776795) (width 0.25) (layer B.Cu) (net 17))
 (segment (start 136.75 43.776795) (end 136.75 45.25) (width 0.25) (layer B.Cu) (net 17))
 (segment (start 133.55 37.94) (end 133.55 40.576795) (width 0.25) (layer B.Cu) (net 17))
 (segment (start 143 48) (end 143 52.765) (width 0.25) (layer B.Cu) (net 5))
 (segment (start 134.72 39.72) (end 143 48) (width 0.25) (layer B.Cu) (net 5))
 (segment (start 143 52.765) (end 143.075 52.84) (width 0.25) (layer B.Cu) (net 5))
 (segment (start 134.57 39.72) (end 134.72 39.72) (width 0.25) (layer B.Cu) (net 5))
 (segment (start 144.46 48.86863) (end 144.46 50) (width 0.25) (layer B.Cu) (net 18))
 (segment (start 144.454999 44.111999) (end 144.454999 48.863629) (width 0.25) (layer B.Cu) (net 18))
 (segment (start 144.454999 48.863629) (end 144.46 48.86863) (width 0.25) (layer B.Cu) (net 18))
 (segment (start 146.43 42.136998) (end 144.454999 44.111999) (width 0.25) (layer B.Cu) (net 18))
 (segment (start 146.43 37.94) (end 146.43 42.136998) (width 0.25) (layer B.Cu) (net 18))
 (segment (start 145.75 52.745) (end 145.845 52.84) (width 0.25) (layer B.Cu) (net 6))
 (segment (start 145.75 47) (end 145.75 52.745) (width 0.25) (layer B.Cu) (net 6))
 (segment (start 147.45 45.3) (end 145.75 47) (width 0.25) (layer B.Cu) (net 6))
 (segment (start 147.45 39.72) (end 147.45 45.3) (width 0.25) (layer B.Cu) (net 6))
 (segment (start 147.25 49.98) (end 147.23 50) (width 0.25) (layer B.Cu) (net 19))
 (segment (start 148.47 45.78) (end 147.25 47) (width 0.25) (layer B.Cu) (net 19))
 (segment (start 147.25 47) (end 147.25 49.98) (width 0.25) (layer B.Cu) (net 19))
 (segment (start 148.47 37.94) (end 148.47 45.78) (width 0.25) (layer B.Cu) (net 19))
 (segment (start 150.84 52.84) (end 151.385 52.84) (width 0.25) (layer F.Cu) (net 8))
 (segment (start 149.49 39.72) (end 149.5 39.73) (width 0.25) (layer F.Cu) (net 8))
 (segment (start 149.5 48.667499) (end 148.75 49.417499) (width 0.25) (layer F.Cu) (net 8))
 (segment (start 149.5 39.73) (end 149.5 48.667499) (width 0.25) (layer F.Cu) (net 8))
 (segment (start 148.75 50.75) (end 150.84 52.84) (width 0.25) (layer F.Cu) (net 8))
 (segment (start 148.75 49.417499) (end 148.75 50.75) (width 0.25) (layer F.Cu) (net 8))
 (segment (start 150.51 49.49) (end 150 50) (width 0.25) (layer F.Cu) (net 20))
 (segment (start 150.51 37.94) (end 150.51 49.49) (width 0.25) (layer F.Cu) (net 20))
 (segment (start 148.75 52.705) (end 148.615 52.84) (width 0.25) (layer B.Cu) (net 7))
 (segment (start 148.75 47.25) (end 148.75 52.705) (width 0.25) (layer B.Cu) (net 7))
 (segment (start 151.53 44.47) (end 148.75 47.25) (width 0.25) (layer B.Cu) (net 7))
 (segment (start 151.53 39.72) (end 151.53 44.47) (width 0.25) (layer B.Cu) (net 7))
 (segment (start 152.5 49.73) (end 152.77 50) (width 0.25) (layer B.Cu) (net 21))
 (segment (start 152.5 40.193002) (end 152.5 49.73) (width 0.25) (layer B.Cu) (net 21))
 (segment (start 152.505001 40.188001) (end 152.5 40.193002) (width 0.25) (layer B.Cu) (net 21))
 (segment (start 152.505001 39.251999) (end 152.505001 40.188001) (width 0.25) (layer B.Cu) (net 21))
 (segment (start 152.5 39.246998) (end 152.505001 39.251999) (width 0.25) (layer B.Cu) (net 21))
 (segment (start 152.5 37.99) (end 152.5 39.246998) (width 0.25) (layer B.Cu) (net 21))
 (segment (start 152.55 37.94) (end 152.5 37.99) (width 0.25) (layer B.Cu) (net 21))
 (segment (start 154 52.685) (end 154.155 52.84) (width 0.25) (layer B.Cu) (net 9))
 (segment (start 154 45.453002) (end 154 52.685) (width 0.25) (layer B.Cu) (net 9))
 (segment (start 153.57 45.023002) (end 154 45.453002) (width 0.25) (layer B.Cu) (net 9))
 (segment (start 153.57 39.72) (end 153.57 45.023002) (width 0.25) (layer B.Cu) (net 9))
 (segment (start 155.5 47.75) (end 155.5 49.96) (width 0.25) (layer B.Cu) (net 22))
 (segment (start 165.31 37.94) (end 155.5 47.75) (width 0.25) (layer B.Cu) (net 22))
 (segment (start 155.5 49.96) (end 155.54 50) (width 0.25) (layer B.Cu) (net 22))
 (segment (start 165.43 37.94) (end 165.31 37.94) (width 0.25) (layer B.Cu) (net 22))
 (segment (start 157 52.765) (end 156.925 52.84) (width 0.25) (layer B.Cu) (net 10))
 (segment (start 157 47.75) (end 157 52.765) (width 0.25) (layer B.Cu) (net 10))
 (segment (start 165.03 39.72) (end 157 47.75) (width 0.25) (layer B.Cu) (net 10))
 (segment (start 166.45 39.72) (end 165.03 39.72) (width 0.25) (layer B.Cu) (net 10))
 (segment (start 159.109999 49.200001) (end 158.31 50) (width 0.25) (layer B.Cu) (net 23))
 (segment (start 163.25 45.06) (end 159.109999 49.200001) (width 0.25) (layer B.Cu) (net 23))
 (segment (start 163.25 44.316998) (end 163.25 45.06) (width 0.25) (layer B.Cu) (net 23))
 (segment (start 167.47 40.096998) (end 163.25 44.316998) (width 0.25) (layer B.Cu) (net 23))
 (segment (start 167.47 37.94) (end 167.47 40.096998) (width 0.25) (layer B.Cu) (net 23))
 (segment (start 162.465 51.70863) (end 162.465 52.84) (width 0.25) (layer F.Cu) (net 12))
 (segment (start 168.5 43.5) (end 162.465 49.535) (width 0.25) (layer F.Cu) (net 12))
 (segment (start 168.5 39.73) (end 168.5 43.5) (width 0.25) (layer F.Cu) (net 12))
 (segment (start 162.465 49.535) (end 162.465 51.70863) (width 0.25) (layer F.Cu) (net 12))
 (segment (start 168.49 39.72) (end 168.5 39.73) (width 0.25) (layer F.Cu) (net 12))
 (segment (start 161 53.25) (end 161 50.08) (width 0.25) (layer F.Cu) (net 24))
 (segment (start 162 54.25) (end 161 53.25) (width 0.25) (layer F.Cu) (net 24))
 (segment (start 161 50.08) (end 161.08 50) (width 0.25) (layer F.Cu) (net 24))
 (segment (start 165.25 50.75) (end 163.75 52.25) (width 0.25) (layer F.Cu) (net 24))
 (segment (start 165.25 49) (end 165.25 50.75) (width 0.25) (layer F.Cu) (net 24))
 (segment (start 169.51 44.74) (end 165.25 49) (width 0.25) (layer F.Cu) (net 24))
 (segment (start 163.75 53.5) (end 163 54.25) (width 0.25) (layer F.Cu) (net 24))
 (segment (start 163.75 52.25) (end 163.75 53.5) (width 0.25) (layer F.Cu) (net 24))
 (segment (start 163 54.25) (end 162 54.25) (width 0.25) (layer F.Cu) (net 24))
 (segment (start 169.51 37.94) (end 169.51 44.74) (width 0.25) (layer F.Cu) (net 24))
 (segment (start 159.75 49.332499) (end 159.75 52.785) (width 0.25) (layer B.Cu) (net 11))
 (segment (start 159.75 52.785) (end 159.695 52.84) (width 0.25) (layer B.Cu) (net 11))
 (segment (start 170.53 39.72) (end 170.53 39.97) (width 0.25) (layer B.Cu) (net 11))
 (segment (start 160.332499 48.75) (end 159.75 49.332499) (width 0.25) (layer B.Cu) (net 11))
 (segment (start 161.75 48.75) (end 160.332499 48.75) (width 0.25) (layer B.Cu) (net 11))
 (segment (start 170.53 39.97) (end 161.75 48.75) (width 0.25) (layer B.Cu) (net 11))
 (segment (start 164 47.75) (end 164 49.85) (width 0.25) (layer B.Cu) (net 25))
 (segment (start 164 49.85) (end 163.85 50) (width 0.25) (layer B.Cu) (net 25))
 (segment (start 171.55 40.2) (end 164 47.75) (width 0.25) (layer B.Cu) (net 25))
 (segment (start 171.55 37.94) (end 171.55 40.2) (width 0.25) (layer B.Cu) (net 25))
 (segment (start 165.235 51.70863) (end 165.235 52.84) (width 0.25) (layer B.Cu) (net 13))
 (segment (start 165.235 47.765) (end 165.235 51.70863) (width 0.25) (layer B.Cu) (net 13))
 (segment (start 172.57 40.43) (end 165.235 47.765) (width 0.25) (layer B.Cu) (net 13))
 (segment (start 172.57 39.72) (end 172.57 40.43) (width 0.25) (layer B.Cu) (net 13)))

